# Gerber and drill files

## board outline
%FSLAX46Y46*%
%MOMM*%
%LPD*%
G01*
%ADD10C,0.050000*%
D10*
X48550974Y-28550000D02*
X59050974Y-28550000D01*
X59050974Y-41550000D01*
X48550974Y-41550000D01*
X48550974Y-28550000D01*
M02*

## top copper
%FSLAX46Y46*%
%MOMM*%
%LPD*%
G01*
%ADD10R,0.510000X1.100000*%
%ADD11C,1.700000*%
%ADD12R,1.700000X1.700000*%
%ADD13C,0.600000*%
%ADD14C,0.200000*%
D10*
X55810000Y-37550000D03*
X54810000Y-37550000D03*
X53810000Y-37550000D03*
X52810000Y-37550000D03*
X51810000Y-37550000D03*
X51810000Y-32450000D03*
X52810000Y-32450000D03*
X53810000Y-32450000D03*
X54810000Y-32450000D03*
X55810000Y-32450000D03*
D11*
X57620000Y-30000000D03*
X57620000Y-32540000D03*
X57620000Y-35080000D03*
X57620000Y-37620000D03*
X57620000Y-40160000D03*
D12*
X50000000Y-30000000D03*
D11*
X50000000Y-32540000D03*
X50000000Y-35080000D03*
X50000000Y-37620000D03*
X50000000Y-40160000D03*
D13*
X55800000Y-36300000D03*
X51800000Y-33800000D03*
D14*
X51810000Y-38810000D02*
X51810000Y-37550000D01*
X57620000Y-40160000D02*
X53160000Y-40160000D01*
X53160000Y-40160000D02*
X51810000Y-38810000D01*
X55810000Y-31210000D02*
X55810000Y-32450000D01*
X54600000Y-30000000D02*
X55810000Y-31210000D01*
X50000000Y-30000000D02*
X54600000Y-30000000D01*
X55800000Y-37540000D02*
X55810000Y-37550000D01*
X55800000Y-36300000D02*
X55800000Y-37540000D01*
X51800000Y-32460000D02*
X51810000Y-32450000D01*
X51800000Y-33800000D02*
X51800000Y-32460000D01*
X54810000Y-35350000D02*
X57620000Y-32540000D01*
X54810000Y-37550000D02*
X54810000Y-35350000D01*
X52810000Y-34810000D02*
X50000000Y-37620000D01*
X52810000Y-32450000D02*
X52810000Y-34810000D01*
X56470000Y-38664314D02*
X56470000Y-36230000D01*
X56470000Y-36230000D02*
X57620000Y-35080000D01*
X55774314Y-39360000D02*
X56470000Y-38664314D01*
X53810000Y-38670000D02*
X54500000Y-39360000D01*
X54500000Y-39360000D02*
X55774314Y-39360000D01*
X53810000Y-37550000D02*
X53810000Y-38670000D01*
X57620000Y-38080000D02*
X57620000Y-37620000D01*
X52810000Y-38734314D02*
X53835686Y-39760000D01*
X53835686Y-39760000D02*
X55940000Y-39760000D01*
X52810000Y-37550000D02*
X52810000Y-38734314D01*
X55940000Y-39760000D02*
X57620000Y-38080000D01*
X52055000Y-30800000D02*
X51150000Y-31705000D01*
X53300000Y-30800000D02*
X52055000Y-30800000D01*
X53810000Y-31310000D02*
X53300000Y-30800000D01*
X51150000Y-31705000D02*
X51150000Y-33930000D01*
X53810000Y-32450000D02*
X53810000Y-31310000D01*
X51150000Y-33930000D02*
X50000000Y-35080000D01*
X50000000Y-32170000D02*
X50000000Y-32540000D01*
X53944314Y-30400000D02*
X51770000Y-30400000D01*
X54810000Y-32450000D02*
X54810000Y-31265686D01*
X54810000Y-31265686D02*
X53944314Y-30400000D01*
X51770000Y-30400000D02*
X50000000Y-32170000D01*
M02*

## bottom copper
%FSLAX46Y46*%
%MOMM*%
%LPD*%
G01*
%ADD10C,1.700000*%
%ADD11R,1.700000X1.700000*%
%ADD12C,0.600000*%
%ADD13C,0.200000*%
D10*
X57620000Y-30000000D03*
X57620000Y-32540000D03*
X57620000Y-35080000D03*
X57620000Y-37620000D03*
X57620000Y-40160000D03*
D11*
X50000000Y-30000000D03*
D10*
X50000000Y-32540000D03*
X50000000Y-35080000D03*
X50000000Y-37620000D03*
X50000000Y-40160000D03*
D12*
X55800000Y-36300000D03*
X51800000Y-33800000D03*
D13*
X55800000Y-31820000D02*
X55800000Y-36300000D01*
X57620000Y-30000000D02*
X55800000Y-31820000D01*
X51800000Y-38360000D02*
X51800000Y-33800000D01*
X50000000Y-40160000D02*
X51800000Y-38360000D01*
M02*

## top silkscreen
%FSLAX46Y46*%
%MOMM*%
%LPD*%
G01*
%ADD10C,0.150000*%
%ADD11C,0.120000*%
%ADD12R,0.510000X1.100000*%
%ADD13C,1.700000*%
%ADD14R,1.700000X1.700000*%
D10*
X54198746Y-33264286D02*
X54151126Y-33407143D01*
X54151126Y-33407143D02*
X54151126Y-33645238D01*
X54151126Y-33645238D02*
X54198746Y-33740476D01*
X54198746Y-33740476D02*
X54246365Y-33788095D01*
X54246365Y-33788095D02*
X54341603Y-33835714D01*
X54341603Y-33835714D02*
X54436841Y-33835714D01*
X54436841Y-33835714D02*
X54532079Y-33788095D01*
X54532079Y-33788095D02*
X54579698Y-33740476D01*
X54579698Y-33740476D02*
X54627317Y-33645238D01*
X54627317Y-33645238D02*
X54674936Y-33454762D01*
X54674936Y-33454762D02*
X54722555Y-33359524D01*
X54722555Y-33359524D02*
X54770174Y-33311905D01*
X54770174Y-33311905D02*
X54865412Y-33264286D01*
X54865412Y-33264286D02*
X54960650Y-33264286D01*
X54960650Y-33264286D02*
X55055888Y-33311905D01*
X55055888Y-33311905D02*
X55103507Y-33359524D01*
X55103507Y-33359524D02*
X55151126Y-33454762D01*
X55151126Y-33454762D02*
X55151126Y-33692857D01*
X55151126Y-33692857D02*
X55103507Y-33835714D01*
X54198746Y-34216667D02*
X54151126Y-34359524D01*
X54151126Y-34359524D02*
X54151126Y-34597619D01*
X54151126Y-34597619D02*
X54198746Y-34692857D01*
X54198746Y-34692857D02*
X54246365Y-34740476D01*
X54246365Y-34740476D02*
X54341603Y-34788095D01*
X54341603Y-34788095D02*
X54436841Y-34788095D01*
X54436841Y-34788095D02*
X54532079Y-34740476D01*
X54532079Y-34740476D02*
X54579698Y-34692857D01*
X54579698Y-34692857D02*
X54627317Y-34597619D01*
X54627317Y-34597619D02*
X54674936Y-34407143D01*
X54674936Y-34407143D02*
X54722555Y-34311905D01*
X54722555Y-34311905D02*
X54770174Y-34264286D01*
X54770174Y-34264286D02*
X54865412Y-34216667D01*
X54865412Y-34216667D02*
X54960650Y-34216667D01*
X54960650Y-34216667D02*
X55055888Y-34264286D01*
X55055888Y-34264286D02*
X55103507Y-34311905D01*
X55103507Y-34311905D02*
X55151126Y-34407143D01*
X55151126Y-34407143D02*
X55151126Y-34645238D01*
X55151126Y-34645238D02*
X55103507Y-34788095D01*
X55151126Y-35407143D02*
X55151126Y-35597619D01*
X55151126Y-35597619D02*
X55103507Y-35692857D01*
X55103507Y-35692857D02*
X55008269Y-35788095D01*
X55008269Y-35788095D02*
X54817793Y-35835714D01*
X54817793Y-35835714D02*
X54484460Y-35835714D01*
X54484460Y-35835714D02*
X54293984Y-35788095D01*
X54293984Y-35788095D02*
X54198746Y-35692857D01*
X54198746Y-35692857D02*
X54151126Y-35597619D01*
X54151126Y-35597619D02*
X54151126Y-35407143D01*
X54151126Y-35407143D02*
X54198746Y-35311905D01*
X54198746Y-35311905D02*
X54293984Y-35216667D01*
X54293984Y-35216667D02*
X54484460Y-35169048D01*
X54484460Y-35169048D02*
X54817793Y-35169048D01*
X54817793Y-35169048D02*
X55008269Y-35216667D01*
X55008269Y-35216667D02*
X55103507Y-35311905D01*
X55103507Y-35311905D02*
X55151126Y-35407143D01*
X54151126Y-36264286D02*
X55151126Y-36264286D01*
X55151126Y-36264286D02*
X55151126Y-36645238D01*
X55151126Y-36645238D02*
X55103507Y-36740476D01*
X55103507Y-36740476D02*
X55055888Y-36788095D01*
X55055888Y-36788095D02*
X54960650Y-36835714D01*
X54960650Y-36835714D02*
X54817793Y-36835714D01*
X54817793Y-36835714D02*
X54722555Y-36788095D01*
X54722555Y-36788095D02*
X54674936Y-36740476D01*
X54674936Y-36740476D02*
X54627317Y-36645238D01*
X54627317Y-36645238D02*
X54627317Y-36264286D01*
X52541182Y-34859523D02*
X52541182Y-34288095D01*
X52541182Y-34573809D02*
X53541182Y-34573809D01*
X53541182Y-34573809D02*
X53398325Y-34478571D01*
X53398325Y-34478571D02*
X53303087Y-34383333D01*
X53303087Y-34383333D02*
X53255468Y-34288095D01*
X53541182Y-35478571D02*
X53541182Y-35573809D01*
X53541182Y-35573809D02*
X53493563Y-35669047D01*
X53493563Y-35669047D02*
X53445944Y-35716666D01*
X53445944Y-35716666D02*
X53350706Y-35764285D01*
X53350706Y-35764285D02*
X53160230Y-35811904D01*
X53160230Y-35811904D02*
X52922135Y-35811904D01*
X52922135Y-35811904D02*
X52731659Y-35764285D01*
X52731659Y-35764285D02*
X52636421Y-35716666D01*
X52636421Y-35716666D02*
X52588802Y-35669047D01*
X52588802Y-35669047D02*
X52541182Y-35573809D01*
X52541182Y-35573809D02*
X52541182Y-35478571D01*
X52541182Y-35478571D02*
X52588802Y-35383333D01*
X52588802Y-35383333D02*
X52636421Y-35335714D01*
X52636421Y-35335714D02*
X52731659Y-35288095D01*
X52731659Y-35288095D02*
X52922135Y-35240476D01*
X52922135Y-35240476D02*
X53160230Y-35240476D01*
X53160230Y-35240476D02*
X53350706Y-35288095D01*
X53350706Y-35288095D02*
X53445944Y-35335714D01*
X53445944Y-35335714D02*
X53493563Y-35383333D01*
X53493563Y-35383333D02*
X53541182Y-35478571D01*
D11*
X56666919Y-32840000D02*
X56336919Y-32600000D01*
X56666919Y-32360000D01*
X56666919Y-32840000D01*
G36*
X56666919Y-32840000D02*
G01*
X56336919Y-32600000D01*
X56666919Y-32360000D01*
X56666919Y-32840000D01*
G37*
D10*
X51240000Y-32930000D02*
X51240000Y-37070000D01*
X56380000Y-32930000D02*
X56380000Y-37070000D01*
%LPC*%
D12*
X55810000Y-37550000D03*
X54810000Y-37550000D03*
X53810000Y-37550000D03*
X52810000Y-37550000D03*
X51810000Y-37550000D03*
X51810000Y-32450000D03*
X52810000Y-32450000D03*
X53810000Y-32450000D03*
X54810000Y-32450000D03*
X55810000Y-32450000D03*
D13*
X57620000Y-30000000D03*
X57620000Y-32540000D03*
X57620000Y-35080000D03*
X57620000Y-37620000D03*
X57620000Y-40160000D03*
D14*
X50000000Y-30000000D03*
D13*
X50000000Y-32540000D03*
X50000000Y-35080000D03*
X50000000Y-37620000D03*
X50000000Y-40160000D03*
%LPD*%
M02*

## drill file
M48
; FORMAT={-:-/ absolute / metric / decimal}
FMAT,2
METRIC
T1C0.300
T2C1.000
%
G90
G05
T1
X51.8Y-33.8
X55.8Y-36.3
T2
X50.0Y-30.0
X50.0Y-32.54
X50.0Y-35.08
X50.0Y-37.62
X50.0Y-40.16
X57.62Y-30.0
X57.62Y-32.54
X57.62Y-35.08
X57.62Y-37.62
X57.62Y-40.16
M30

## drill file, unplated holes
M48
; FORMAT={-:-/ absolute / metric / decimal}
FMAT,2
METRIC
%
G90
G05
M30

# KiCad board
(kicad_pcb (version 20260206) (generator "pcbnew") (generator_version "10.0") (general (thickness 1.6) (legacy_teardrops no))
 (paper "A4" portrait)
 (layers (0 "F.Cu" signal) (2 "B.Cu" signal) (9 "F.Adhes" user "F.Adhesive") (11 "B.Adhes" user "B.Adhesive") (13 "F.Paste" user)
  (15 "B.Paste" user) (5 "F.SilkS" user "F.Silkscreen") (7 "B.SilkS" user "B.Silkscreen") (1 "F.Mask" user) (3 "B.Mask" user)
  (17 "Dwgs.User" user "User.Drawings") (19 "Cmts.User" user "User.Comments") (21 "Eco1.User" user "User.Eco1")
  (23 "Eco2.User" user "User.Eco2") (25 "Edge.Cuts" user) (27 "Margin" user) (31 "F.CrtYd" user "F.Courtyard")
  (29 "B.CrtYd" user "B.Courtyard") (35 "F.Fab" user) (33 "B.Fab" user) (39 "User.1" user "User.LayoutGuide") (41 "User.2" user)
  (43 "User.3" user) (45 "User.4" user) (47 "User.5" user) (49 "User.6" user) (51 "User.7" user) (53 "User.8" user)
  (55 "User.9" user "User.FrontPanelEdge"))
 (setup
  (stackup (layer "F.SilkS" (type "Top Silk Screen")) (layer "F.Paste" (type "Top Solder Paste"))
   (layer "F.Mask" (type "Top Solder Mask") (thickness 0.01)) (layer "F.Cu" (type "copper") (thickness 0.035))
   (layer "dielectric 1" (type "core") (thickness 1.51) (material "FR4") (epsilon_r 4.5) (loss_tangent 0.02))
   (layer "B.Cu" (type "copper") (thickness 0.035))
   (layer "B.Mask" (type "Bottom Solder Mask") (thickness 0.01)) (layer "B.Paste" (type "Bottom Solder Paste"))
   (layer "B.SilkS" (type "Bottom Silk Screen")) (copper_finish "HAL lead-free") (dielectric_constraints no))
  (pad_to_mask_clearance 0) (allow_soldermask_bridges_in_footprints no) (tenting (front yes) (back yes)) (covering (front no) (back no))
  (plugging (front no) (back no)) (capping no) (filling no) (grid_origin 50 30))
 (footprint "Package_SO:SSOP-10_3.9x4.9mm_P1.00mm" (layer "F.Cu") (at 53.81 35 -90)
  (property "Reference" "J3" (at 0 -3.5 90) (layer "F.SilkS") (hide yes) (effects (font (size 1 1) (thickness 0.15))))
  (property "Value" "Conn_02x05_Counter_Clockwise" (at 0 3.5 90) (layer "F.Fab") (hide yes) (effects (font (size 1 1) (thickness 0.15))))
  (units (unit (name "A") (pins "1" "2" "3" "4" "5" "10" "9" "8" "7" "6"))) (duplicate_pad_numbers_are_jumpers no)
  (fp_line (start -2.07 2.57) (end 2.07 2.57) (stroke (width 0.15) (type solid)) (layer "F.SilkS"))
  (fp_line (start -2.07 -2.57) (end 2.07 -2.57) (stroke (width 0.15) (type solid)) (layer "F.SilkS"))
  (fp_poly
   (pts (xy -2.4 -2.526919) (xy -2.64 -2.856919) (xy -2.16 -2.856919) (xy -2.4 -2.526919)) (stroke (width 0.12) (type solid)) (fill yes)
   (layer "F.SilkS"))
  (pad "1" smd rect (at -2.55 -2 270) (size 1.1 0.51) (layers "F.Cu" "F.Mask" "F.Paste") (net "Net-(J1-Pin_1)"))
  (pad "2" smd rect (at -2.55 -1 270) (size 1.1 0.51) (layers "F.Cu" "F.Mask" "F.Paste") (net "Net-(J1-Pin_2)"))
  (pad "3" smd rect (at -2.55 0 270) (size 1.1 0.51) (layers "F.Cu" "F.Mask" "F.Paste") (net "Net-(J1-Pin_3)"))
  (pad "4" smd rect (at -2.55 1 270) (size 1.1 0.51) (layers "F.Cu" "F.Mask" "F.Paste") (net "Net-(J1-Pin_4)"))
  (pad "5" smd rect (at -2.55 2 270) (size 1.1 0.51) (layers "F.Cu" "F.Mask" "F.Paste") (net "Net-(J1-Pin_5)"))
  (pad "6" smd rect (at 2.55 2 270) (size 1.1 0.51) (layers "F.Cu" "F.Mask" "F.Paste") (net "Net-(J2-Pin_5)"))
  (pad "7" smd rect (at 2.55 1 270) (size 1.1 0.51) (layers "F.Cu" "F.Mask" "F.Paste") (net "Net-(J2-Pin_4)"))
  (pad "8" smd rect (at 2.55 0 270) (size 1.1 0.51) (layers "F.Cu" "F.Mask" "F.Paste") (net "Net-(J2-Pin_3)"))
  (pad "9" smd rect (at 2.55 -1 270) (size 1.1 0.51) (layers "F.Cu" "F.Mask" "F.Paste") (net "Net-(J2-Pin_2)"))
  (pad "10" smd rect (at 2.55 -2 270) (size 1.1 0.51) (layers "F.Cu" "F.Mask" "F.Paste") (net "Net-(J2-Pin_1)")))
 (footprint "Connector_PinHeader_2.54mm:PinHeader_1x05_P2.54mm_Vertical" (layer "B.Cu") (at 50 30 180)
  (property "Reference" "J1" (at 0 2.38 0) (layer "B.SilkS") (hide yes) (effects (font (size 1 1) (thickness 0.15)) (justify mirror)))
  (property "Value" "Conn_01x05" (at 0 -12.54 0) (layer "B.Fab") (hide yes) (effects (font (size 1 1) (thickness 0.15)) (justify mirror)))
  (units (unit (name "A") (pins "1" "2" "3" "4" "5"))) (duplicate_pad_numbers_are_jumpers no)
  (pad "1" thru_hole rect (at 0 0 180) (size 1.7 1.7) (drill 1) (layers "*.Cu" "*.Mask") (remove_unused_layers no) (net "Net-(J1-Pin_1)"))
  (pad "2" thru_hole circle (at 0 -2.54 180) (size 1.7 1.7) (drill 1) (layers "*.Cu" "*.Mask") (remove_unused_layers no)
   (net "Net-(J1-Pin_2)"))
  (pad "3" thru_hole circle (at 0 -5.08 180) (size 1.7 1.7) (drill 1) (layers "*.Cu" "*.Mask") (remove_unused_layers no)
   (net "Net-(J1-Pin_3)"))
  (pad "4" thru_hole circle (at 0 -7.62 180) (size 1.7 1.7) (drill 1) (layers "*.Cu" "*.Mask") (remove_unused_layers no)
   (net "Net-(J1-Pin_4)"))
  (pad "5" thru_hole circle (at 0 -10.16 180) (size 1.7 1.7) (drill 1) (layers "*.Cu" "*.Mask") (remove_unused_layers no)
   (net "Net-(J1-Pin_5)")))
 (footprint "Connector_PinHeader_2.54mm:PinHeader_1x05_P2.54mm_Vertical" (layer "B.Cu") (at 57.62 30 180)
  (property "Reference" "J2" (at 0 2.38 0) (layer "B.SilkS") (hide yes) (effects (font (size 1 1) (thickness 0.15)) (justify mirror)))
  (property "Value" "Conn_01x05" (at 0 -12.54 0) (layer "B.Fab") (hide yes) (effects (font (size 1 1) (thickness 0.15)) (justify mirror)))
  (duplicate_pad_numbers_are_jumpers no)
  (pad "1" thru_hole circle (at 0 0 180) (size 1.7 1.7) (drill 1) (layers "*.Cu" "*.Mask") (remove_unused_layers no) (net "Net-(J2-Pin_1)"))
  (pad "2" thru_hole circle (at 0 -2.54 180) (size 1.7 1.7) (drill 1) (layers "*.Cu" "*.Mask") (remove_unused_layers no)
   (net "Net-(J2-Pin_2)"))
  (pad "3" thru_hole circle (at 0 -5.08 180) (size 1.7 1.7) (drill 1) (layers "*.Cu" "*.Mask") (remove_unused_layers no)
   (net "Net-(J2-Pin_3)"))
  (pad "4" thru_hole circle (at 0 -7.62 180) (size 1.7 1.7) (drill 1) (layers "*.Cu" "*.Mask") (remove_unused_layers no)
   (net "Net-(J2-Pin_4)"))
  (pad "5" thru_hole circle (at 0 -10.16 180) (size 1.7 1.7) (drill 1) (layers "*.Cu" "*.Mask") (remove_unused_layers no)
   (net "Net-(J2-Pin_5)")))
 (gr_rect (start 48.550974 28.55) (end 59.050974 41.55) (stroke (width 0.05) (type solid)) (fill no) (layer "Edge.Cuts"))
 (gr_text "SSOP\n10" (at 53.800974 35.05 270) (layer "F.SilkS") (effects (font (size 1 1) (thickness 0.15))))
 (segment (start 54.6 30) (end 55.81 31.21) (width 0.2) (layer "F.Cu") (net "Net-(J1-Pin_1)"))
 (segment (start 55.81 31.21) (end 55.81 32.45) (width 0.2) (layer "F.Cu") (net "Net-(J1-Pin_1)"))
 (segment (start 50 30) (end 54.6 30) (width 0.2) (layer "F.Cu") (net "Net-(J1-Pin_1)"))
 (segment (start 50 32.17) (end 50 32.54) (width 0.2) (layer "F.Cu") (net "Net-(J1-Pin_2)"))
 (segment (start 54.81 31.265686) (end 53.944314 30.4) (width 0.2) (layer "F.Cu") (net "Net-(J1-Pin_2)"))
 (segment (start 54.81 32.45) (end 54.81 31.265686) (width 0.2) (layer "F.Cu") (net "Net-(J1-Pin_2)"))
 (segment (start 51.77 30.4) (end 50 32.17) (width 0.2) (layer "F.Cu") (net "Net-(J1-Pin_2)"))
 (segment (start 53.944314 30.4) (end 51.77 30.4) (width 0.2) (layer "F.Cu") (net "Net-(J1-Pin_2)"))
 (segment (start 53.81 31.31) (end 53.3 30.8) (width 0.2) (layer "F.Cu") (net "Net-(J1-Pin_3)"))
 (segment (start 52.055 30.8) (end 51.15 31.705) (width 0.2) (layer "F.Cu") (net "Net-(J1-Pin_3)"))
 (segment (start 53.81 32.45) (end 53.81 31.31) (width 0.2) (layer "F.Cu") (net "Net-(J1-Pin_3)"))
 (segment (start 51.15 31.705) (end 51.15 33.93) (width 0.2) (layer "F.Cu") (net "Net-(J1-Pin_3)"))
 (segment (start 53.3 30.8) (end 52.055 30.8) (width 0.2) (layer "F.Cu") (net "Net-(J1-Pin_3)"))
 (segment (start 51.15 33.93) (end 50 35.08) (width 0.2) (layer "F.Cu") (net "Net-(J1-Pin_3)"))
 (segment (start 52.81 34.81) (end 50 37.62) (width 0.2) (layer "F.Cu") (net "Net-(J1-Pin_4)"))
 (segment (start 52.81 32.45) (end 52.81 34.81) (width 0.2) (layer "F.Cu") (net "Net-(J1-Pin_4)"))
 (segment (start 51.8 33.8) (end 51.8 32.46) (width 0.2) (layer "F.Cu") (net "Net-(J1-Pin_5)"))
 (segment (start 51.8 32.46) (end 51.81 32.45) (width 0.2) (layer "F.Cu") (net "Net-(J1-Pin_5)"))
 (via (at 51.8 33.8) (size 0.6) (drill 0.3) (layers "F.Cu" "B.Cu") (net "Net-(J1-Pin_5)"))
 (segment (start 51.8 38.36) (end 51.8 33.8) (width 0.2) (layer "B.Cu") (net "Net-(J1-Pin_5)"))
 (segment (start 50 40.16) (end 51.8 38.36) (width 0.2) (layer "B.Cu") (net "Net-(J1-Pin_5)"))
 (segment (start 57.62 40.16) (end 53.16 40.16) (width 0.2) (layer "F.Cu") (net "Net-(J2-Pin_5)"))
 (segment (start 51.81 38.81) (end 51.81 37.55) (width 0.2) (layer "F.Cu") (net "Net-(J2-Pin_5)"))
 (segment (start 53.16 40.16) (end 51.81 38.81) (width 0.2) (layer "F.Cu") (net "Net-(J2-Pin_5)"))
 (segment (start 53.835686 39.76) (end 55.94 39.76) (width 0.2) (layer "F.Cu") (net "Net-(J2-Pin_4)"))
 (segment (start 55.94 39.76) (end 57.62 38.08) (width 0.2) (layer "F.Cu") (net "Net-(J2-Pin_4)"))
 (segment (start 52.81 38.734314) (end 53.835686 39.76) (width 0.2) (layer "F.Cu") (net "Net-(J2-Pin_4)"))
 (segment (start 52.81 37.55) (end 52.81 38.734314) (width 0.2) (layer "F.Cu") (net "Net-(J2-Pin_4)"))
 (segment (start 57.62 38.08) (end 57.62 37.62) (width 0.2) (layer "F.Cu") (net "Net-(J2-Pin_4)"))
 (segment (start 53.81 38.67) (end 54.5 39.36) (width 0.2) (layer "F.Cu") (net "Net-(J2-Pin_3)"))
 (segment (start 54.5 39.36) (end 55.774314 39.36) (width 0.2) (layer "F.Cu") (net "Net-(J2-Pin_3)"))
 (segment (start 56.47 36.23) (end 57.62 35.08) (width 0.2) (layer "F.Cu") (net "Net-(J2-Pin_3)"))
 (segment (start 53.81 37.55) (end 53.81 38.67) (width 0.2) (layer "F.Cu") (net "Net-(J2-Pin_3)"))
 (segment (start 56.47 38.664314) (end 56.47 36.23) (width 0.2) (layer "F.Cu") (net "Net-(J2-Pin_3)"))
 (segment (start 55.774314 39.36) (end 56.47 38.664314) (width 0.2) (layer "F.Cu") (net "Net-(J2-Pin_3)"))
 (segment (start 54.81 35.35) (end 57.62 32.54) (width 0.2) (layer "F.Cu") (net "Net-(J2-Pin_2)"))
 (segment (start 54.81 37.55) (end 54.81 35.35) (width 0.2) (layer "F.Cu") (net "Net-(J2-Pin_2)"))
 (segment (start 55.8 36.3) (end 55.8 37.54) (width 0.2) (layer "F.Cu") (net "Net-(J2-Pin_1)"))
 (segment (start 55.8 37.54) (end 55.81 37.55) (width 0.2) (layer "F.Cu") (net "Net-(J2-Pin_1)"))
 (via (at 55.8 36.3) (size 0.6) (drill 0.3) (layers "F.Cu" "B.Cu") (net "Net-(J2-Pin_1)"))
 (segment (start 55.8 31.82) (end 55.8 36.3) (width 0.2) (layer "B.Cu") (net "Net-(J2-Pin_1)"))
 (segment (start 57.62 30) (end 55.8 31.82) (width 0.2) (layer "B.Cu") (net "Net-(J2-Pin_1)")))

